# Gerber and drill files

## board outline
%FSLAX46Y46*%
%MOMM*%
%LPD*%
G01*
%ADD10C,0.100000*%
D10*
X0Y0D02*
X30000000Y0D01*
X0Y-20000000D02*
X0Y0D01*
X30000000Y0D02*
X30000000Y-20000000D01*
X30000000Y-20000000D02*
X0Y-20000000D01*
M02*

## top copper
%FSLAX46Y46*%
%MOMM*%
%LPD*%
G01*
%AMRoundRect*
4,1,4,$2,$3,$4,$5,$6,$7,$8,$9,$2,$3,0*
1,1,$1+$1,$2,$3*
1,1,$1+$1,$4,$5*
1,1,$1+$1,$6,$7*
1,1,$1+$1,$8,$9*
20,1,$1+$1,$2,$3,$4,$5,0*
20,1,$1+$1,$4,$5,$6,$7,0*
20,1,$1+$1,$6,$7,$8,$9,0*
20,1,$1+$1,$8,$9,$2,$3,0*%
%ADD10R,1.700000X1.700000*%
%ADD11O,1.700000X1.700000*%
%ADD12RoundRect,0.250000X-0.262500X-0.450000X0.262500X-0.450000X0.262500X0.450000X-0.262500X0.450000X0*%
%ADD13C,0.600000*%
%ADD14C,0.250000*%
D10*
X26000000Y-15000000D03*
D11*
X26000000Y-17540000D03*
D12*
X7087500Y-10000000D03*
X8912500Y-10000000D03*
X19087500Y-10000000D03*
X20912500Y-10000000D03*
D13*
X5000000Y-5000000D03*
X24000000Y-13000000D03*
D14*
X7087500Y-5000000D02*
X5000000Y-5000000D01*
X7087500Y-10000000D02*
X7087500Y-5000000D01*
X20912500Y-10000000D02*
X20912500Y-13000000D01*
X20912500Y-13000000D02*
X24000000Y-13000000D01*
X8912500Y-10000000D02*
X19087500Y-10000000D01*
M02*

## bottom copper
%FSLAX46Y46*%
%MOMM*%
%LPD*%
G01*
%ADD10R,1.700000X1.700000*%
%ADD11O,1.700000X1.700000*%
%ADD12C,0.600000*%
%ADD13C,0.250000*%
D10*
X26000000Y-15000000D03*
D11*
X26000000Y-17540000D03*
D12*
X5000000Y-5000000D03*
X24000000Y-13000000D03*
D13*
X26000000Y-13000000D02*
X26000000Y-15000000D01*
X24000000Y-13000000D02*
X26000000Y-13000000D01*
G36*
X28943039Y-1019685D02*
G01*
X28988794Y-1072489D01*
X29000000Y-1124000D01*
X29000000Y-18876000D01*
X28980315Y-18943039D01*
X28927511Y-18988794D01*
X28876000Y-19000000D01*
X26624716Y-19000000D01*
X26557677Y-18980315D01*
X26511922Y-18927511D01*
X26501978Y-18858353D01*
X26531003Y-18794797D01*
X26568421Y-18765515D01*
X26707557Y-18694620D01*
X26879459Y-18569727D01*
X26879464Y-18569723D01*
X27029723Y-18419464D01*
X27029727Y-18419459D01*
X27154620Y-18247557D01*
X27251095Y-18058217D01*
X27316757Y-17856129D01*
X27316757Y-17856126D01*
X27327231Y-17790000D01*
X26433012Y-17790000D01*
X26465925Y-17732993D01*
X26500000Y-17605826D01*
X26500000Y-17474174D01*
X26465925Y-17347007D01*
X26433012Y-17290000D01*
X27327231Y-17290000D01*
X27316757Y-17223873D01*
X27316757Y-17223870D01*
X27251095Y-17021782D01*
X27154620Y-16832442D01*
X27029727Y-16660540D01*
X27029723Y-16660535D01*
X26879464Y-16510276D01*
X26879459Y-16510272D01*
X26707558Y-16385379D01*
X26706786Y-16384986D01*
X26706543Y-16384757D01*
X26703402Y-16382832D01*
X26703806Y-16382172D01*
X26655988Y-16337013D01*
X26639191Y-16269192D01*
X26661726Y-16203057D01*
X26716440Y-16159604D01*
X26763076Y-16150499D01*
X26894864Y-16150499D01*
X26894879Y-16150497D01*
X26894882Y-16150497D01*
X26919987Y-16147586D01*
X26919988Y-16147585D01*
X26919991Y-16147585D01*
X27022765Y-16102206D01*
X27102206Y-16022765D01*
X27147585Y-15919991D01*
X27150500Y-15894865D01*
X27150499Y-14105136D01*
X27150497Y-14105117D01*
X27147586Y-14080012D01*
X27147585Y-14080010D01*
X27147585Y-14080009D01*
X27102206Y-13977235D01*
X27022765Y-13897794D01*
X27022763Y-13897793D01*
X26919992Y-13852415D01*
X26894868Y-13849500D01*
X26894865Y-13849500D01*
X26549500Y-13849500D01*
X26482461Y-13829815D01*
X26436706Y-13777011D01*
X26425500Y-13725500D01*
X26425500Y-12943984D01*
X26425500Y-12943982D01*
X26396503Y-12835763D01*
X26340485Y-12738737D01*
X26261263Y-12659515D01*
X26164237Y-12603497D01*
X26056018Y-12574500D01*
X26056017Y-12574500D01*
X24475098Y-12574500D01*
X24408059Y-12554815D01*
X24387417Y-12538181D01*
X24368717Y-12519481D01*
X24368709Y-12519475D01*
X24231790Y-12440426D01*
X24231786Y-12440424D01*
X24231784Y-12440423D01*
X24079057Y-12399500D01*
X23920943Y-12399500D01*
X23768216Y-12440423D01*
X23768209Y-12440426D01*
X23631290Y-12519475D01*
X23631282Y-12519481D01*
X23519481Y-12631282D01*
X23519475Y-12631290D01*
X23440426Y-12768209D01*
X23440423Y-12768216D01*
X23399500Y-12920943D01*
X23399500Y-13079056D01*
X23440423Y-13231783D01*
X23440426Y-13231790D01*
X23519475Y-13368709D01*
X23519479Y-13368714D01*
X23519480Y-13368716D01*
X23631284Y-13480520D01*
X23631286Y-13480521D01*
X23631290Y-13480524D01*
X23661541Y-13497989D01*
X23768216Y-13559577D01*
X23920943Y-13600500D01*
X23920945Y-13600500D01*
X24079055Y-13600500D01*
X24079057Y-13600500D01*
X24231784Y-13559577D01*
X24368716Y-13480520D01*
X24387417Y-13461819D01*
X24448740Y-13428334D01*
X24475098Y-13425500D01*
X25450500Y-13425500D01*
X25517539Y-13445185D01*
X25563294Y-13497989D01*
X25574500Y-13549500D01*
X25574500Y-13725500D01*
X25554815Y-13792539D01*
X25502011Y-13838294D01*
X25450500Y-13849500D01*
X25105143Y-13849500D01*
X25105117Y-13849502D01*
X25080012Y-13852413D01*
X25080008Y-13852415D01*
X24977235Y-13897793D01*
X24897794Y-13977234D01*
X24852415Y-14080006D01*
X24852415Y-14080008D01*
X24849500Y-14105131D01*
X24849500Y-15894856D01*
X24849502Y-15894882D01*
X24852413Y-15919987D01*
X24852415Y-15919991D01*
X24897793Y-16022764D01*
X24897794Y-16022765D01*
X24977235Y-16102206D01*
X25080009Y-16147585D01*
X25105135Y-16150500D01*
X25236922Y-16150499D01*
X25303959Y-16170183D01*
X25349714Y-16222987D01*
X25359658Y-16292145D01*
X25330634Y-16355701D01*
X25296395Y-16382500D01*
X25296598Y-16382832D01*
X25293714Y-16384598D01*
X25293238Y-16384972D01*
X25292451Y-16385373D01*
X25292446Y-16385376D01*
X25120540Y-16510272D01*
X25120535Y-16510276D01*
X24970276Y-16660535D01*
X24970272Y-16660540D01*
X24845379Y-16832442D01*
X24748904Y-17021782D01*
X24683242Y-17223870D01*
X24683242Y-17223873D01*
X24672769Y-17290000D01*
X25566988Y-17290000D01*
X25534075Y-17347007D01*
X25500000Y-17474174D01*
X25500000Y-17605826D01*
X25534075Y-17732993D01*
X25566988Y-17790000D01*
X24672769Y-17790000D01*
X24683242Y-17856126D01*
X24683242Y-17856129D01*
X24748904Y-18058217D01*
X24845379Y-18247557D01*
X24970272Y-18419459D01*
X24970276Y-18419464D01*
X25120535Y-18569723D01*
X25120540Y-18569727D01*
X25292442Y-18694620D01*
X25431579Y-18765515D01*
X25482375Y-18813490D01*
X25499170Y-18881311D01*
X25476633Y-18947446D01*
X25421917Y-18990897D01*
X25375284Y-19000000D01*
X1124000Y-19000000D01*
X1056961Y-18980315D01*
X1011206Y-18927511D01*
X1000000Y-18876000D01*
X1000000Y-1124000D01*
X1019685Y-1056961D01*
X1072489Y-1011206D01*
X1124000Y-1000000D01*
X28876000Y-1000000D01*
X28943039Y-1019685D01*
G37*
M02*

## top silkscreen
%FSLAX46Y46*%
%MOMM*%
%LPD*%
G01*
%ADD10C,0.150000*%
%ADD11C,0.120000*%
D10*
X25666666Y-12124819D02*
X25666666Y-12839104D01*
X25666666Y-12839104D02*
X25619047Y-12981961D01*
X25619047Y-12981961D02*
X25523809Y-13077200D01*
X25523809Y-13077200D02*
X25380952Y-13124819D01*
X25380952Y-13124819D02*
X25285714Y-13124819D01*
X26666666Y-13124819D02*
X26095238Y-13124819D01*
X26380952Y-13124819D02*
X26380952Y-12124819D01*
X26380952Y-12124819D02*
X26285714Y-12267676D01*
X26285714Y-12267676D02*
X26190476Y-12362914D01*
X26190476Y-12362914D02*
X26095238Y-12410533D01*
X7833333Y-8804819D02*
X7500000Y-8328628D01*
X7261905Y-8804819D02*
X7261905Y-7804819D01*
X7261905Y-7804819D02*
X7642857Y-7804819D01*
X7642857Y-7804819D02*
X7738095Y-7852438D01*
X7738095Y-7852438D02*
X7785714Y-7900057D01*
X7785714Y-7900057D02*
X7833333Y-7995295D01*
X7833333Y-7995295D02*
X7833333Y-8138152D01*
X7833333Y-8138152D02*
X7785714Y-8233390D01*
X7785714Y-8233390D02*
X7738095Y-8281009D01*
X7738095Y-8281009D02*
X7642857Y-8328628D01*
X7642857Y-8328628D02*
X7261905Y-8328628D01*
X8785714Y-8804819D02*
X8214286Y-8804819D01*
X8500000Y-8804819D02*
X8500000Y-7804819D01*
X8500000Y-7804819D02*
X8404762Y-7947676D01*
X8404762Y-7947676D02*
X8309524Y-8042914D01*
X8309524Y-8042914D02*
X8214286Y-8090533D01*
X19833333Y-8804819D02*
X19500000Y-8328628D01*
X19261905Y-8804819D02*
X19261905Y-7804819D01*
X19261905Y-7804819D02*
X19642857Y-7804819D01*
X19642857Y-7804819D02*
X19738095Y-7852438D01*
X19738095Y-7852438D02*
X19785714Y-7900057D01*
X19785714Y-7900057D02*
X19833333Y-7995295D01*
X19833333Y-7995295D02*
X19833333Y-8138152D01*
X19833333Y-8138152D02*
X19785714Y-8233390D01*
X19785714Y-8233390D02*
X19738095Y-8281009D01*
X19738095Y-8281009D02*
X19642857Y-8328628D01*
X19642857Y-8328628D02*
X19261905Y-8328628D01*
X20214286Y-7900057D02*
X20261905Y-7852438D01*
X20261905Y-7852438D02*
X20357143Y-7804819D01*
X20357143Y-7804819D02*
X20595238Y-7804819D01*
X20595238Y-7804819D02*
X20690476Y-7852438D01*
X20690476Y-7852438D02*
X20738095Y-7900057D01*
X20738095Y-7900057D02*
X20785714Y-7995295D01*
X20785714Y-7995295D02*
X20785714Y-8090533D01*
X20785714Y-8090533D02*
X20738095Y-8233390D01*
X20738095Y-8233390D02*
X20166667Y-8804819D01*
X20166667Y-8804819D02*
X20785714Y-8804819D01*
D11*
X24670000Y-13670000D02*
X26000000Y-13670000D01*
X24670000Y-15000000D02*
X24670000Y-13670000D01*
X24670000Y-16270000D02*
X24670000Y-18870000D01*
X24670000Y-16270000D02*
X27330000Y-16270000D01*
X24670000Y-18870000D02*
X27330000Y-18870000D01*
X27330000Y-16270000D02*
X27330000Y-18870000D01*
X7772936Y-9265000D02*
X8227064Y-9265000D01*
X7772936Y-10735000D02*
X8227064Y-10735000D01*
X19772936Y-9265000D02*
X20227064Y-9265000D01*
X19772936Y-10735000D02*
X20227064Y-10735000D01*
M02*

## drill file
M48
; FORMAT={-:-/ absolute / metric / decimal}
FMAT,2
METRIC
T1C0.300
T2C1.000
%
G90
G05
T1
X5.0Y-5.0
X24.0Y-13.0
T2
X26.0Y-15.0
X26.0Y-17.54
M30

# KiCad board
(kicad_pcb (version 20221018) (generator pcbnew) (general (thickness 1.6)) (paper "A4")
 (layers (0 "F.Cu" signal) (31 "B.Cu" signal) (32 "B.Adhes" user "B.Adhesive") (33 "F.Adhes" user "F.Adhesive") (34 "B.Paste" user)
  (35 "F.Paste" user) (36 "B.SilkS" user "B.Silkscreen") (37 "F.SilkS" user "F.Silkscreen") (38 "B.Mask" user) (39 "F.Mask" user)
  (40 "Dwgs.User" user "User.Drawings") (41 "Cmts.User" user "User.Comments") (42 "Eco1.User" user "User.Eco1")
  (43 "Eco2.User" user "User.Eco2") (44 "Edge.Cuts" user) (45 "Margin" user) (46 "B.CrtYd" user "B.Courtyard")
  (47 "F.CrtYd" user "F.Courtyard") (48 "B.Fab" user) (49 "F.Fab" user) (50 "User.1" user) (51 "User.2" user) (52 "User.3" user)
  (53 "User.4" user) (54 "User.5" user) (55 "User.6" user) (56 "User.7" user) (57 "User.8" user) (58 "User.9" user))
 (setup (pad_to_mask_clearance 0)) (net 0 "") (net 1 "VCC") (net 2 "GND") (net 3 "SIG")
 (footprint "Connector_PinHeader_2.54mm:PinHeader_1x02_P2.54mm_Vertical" (layer "F.Cu") (at 26 15)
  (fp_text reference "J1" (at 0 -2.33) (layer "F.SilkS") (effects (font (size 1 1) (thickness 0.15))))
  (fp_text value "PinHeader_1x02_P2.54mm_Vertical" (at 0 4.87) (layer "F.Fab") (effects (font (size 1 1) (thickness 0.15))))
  (fp_line (start -1.33 -1.33) (end 0 -1.33) (stroke (width 0.12) (type solid)) (layer "F.SilkS"))
  (fp_line (start -1.33 0) (end -1.33 -1.33) (stroke (width 0.12) (type solid)) (layer "F.SilkS"))
  (fp_line (start -1.33 1.27) (end -1.33 3.87) (stroke (width 0.12) (type solid)) (layer "F.SilkS"))
  (fp_line (start -1.33 1.27) (end 1.33 1.27) (stroke (width 0.12) (type solid)) (layer "F.SilkS"))
  (fp_line (start -1.33 3.87) (end 1.33 3.87) (stroke (width 0.12) (type solid)) (layer "F.SilkS"))
  (fp_line (start 1.33 1.27) (end 1.33 3.87) (stroke (width 0.12) (type solid)) (layer "F.SilkS"))
  (pad "1" thru_hole rect (at 0 0) (size 1.7 1.7) (drill 1) (layers "*.Cu" "*.Mask") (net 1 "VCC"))
  (pad "2" thru_hole oval (at 0 2.54) (size 1.7 1.7) (drill 1) (layers "*.Cu" "*.Mask") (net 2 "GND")))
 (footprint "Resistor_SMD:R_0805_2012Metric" (layer "F.Cu") (at 8 10)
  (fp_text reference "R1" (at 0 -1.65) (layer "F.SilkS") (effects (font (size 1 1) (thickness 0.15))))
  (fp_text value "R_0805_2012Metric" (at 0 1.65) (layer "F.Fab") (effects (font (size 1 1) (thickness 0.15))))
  (fp_line (start -0.227064 -0.735) (end 0.227064 -0.735) (stroke (width 0.12) (type solid)) (layer "F.SilkS"))
  (fp_line (start -0.227064 0.735) (end 0.227064 0.735) (stroke (width 0.12) (type solid)) (layer "F.SilkS"))
  (pad "1" smd roundrect (at -0.9125 0) (size 1.025 1.4) (layers "F.Cu" "F.Paste" "F.Mask") (roundrect_rratio 0.243902) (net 2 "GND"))
  (pad "2" smd roundrect (at 0.9125 0) (size 1.025 1.4) (layers "F.Cu" "F.Paste" "F.Mask") (roundrect_rratio 0.243902) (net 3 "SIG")))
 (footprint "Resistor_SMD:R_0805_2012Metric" (layer "F.Cu") (at 20 10)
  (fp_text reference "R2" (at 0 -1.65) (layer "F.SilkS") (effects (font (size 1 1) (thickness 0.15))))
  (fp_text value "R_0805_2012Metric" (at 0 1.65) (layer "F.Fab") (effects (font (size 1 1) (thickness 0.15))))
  (fp_line (start -0.227064 -0.735) (end 0.227064 -0.735) (stroke (width 0.12) (type solid)) (layer "F.SilkS"))
  (fp_line (start -0.227064 0.735) (end 0.227064 0.735) (stroke (width 0.12) (type solid)) (layer "F.SilkS"))
  (pad "1" smd roundrect (at -0.9125 0) (size 1.025 1.4) (layers "F.Cu" "F.Paste" "F.Mask") (roundrect_rratio 0.243902) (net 3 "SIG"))
  (pad "2" smd roundrect (at 0.9125 0) (size 1.025 1.4) (layers "F.Cu" "F.Paste" "F.Mask") (roundrect_rratio 0.243902) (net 1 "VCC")))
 (gr_line (start 0 0) (end 30 0) (stroke (width 0.1) (type default)) (layer "Edge.Cuts"))
 (gr_line (start 0 20) (end 0 0) (stroke (width 0.1) (type default)) (layer "Edge.Cuts"))
 (gr_line (start 30 0) (end 30 20) (stroke (width 0.1) (type default)) (layer "Edge.Cuts"))
 (gr_line (start 30 20) (end 0 20) (stroke (width 0.1) (type default)) (layer "Edge.Cuts"))
 (segment (start 7.0875 5) (end 5 5) (width 0.25) (layer "F.Cu") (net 2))
 (segment (start 7.0875 10) (end 7.0875 5) (width 0.25) (layer "F.Cu") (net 2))
 (via (at 5 5) (size 0.6) (drill 0.3) (layers "F.Cu" "B.Cu") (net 2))
 (segment (start 20.9125 10) (end 20.9125 13) (width 0.25) (layer "F.Cu") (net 1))
 (segment (start 20.9125 13) (end 24 13) (width 0.25) (layer "F.Cu") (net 1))
 (via (at 24 13) (size 0.6) (drill 0.3) (layers "F.Cu" "B.Cu") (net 1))
 (segment (start 26 13) (end 26 15) (width 0.25) (layer "B.Cu") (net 1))
 (segment (start 24 13) (end 26 13) (width 0.25) (layer "B.Cu") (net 1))
 (segment (start 8.9125 10) (end 19.0875 10) (width 0.25) (layer "F.Cu") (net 3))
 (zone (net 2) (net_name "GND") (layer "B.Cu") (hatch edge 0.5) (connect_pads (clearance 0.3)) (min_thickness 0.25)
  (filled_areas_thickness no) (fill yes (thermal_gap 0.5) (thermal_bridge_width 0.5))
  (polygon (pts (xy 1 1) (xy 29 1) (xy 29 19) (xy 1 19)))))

